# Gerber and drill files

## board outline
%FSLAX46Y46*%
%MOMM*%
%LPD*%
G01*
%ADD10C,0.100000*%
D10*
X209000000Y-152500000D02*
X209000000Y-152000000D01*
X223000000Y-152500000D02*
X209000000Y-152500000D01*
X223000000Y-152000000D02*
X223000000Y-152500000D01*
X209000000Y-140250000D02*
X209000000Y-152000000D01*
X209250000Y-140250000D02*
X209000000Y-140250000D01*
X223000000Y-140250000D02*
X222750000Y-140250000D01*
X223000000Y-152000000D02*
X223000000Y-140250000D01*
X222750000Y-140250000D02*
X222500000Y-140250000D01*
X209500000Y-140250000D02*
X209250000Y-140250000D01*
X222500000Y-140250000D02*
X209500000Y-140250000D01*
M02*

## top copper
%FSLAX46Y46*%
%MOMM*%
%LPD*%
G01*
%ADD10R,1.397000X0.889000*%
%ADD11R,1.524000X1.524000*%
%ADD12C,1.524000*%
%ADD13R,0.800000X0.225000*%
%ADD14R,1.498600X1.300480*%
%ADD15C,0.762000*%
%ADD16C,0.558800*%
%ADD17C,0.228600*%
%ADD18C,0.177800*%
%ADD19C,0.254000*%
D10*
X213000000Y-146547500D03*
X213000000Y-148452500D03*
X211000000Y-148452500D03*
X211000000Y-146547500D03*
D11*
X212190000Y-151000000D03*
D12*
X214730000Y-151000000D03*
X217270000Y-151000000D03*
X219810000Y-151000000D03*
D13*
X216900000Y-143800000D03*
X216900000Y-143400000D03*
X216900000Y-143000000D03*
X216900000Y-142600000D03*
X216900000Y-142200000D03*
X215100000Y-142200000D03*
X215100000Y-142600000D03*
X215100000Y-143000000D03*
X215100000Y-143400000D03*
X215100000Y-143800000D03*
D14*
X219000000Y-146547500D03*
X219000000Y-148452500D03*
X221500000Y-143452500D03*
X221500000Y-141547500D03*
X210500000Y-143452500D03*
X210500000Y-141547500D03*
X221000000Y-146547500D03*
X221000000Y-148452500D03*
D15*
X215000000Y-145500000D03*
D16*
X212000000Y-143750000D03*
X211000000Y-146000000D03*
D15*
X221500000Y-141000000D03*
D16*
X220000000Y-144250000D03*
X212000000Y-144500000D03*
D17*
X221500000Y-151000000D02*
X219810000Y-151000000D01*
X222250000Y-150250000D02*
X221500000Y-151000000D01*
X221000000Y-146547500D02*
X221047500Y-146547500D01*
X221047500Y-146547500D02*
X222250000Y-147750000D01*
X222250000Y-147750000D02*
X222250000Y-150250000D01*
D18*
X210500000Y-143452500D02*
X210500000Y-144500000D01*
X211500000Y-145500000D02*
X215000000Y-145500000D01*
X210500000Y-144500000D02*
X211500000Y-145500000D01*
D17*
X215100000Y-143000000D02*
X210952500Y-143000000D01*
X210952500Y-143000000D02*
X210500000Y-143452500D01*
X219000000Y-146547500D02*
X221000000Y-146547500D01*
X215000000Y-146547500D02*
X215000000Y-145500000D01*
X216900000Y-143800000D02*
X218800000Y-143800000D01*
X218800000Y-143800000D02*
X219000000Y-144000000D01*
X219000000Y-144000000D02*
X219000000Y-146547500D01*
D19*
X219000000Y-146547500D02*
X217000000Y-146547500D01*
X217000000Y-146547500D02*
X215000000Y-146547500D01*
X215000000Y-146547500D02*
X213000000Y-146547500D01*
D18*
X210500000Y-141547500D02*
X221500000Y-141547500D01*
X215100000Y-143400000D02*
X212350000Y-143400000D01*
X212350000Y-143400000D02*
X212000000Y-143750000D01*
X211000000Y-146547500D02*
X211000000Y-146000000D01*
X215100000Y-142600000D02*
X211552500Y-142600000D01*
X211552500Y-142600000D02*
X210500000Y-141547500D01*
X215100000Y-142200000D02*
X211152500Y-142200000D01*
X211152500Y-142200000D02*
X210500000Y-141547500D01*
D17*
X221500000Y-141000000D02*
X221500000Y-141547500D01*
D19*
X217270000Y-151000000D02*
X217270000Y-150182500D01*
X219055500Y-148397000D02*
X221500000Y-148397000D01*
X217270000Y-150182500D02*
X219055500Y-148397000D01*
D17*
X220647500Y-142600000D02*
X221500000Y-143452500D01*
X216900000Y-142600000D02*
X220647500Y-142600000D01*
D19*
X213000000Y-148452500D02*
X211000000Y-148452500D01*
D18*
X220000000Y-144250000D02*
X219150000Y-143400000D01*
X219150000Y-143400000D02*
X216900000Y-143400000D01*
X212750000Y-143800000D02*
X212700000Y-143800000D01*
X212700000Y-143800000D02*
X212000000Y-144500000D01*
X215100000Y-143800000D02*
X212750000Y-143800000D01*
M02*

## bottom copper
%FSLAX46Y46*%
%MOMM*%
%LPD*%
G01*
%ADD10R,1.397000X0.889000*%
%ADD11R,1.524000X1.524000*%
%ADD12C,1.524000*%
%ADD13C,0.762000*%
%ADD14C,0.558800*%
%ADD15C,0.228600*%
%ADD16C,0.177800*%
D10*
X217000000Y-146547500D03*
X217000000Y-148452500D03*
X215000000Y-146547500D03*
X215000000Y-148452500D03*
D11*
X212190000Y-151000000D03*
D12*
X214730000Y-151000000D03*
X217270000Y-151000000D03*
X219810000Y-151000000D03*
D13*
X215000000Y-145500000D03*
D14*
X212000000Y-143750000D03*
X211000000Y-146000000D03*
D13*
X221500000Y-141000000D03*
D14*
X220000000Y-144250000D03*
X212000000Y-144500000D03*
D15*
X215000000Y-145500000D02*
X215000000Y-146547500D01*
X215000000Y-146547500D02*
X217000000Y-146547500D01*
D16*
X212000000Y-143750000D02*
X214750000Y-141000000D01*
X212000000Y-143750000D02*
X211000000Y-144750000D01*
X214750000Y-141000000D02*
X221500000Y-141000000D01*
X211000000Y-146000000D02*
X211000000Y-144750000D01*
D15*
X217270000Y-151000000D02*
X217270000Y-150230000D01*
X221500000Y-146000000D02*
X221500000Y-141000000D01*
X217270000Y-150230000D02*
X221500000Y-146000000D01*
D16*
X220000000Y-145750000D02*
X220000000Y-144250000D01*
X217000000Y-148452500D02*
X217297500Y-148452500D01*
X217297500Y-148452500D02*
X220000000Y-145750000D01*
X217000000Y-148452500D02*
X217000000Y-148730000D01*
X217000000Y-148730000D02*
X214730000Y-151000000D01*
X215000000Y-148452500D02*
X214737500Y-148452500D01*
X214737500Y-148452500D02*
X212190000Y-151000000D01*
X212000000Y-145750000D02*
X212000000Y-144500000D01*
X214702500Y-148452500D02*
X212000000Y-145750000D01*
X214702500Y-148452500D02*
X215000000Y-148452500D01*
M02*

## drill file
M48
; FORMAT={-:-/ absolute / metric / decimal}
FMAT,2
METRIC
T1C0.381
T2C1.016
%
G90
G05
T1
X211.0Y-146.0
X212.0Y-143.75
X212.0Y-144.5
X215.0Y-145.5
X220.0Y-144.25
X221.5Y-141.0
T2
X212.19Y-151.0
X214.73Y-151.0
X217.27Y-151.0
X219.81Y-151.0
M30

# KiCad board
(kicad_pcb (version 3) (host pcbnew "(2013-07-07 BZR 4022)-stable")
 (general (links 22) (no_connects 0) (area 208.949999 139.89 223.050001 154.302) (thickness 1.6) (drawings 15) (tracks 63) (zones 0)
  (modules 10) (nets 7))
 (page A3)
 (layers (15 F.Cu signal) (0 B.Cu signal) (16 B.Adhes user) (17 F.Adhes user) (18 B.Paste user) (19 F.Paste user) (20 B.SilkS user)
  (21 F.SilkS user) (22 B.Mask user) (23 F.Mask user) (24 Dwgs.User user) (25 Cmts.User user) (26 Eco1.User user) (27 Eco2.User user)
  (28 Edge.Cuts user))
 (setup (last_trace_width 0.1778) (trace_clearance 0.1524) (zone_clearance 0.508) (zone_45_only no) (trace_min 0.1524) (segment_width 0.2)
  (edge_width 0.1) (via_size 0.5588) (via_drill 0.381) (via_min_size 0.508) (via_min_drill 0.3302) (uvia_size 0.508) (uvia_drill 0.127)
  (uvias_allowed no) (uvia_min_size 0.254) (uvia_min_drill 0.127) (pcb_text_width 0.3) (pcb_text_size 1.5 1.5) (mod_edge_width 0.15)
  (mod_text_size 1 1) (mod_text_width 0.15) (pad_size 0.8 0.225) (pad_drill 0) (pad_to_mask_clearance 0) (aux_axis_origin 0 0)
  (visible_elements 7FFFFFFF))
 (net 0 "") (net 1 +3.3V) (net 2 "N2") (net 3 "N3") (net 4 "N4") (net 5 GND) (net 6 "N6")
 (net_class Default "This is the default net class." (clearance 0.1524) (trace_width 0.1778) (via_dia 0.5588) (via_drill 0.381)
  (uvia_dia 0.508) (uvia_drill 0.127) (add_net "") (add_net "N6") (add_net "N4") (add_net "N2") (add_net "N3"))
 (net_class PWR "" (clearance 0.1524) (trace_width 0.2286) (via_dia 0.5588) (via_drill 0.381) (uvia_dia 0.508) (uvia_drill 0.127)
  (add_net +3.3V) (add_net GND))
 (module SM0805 (layer B.Cu) (at 217 147.5 270)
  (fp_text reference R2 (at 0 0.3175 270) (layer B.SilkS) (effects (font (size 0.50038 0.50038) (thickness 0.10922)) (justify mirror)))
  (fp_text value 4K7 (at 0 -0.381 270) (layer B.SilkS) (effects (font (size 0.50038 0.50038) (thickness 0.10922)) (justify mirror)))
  (pad 1 smd rect (at -0.9525 0 270) (size 0.889 1.397) (layers B.Cu B.Paste B.Mask) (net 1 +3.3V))
  (pad 2 smd rect (at 0.9525 0 270) (size 0.889 1.397) (layers B.Cu B.Paste B.Mask) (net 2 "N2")))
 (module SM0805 (layer B.Cu) (at 215 147.5 270)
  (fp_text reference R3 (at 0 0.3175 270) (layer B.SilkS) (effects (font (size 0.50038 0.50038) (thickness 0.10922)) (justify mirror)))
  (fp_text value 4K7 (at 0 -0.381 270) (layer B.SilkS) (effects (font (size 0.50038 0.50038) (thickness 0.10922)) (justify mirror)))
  (pad 1 smd rect (at -0.9525 0 270) (size 0.889 1.397) (layers B.Cu B.Paste B.Mask) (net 1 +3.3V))
  (pad 2 smd rect (at 0.9525 0 270) (size 0.889 1.397) (layers B.Cu B.Paste B.Mask) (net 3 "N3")))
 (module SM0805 (layer F.Cu) (at 213 147.5 270)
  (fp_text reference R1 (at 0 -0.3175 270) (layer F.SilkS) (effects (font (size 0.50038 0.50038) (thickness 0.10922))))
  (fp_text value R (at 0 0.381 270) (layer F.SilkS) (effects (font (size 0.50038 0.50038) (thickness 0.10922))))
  (pad 1 smd rect (at -0.9525 0 270) (size 0.889 1.397) (layers F.Cu F.Paste F.Mask) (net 1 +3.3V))
  (pad 2 smd rect (at 0.9525 0 270) (size 0.889 1.397) (layers F.Cu F.Paste F.Mask) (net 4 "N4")))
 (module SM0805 (layer F.Cu) (at 211 147.5 90)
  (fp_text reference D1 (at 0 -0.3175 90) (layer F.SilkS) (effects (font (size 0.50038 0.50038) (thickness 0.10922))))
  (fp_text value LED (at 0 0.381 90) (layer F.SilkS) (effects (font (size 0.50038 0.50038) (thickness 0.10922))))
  (pad 1 smd rect (at -0.9525 0 90) (size 0.889 1.397) (layers F.Cu F.Paste F.Mask) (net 4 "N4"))
  (pad 2 smd rect (at 0.9525 0 90) (size 0.889 1.397) (layers F.Cu F.Paste F.Mask) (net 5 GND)))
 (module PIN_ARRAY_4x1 (layer F.Cu) (at 216 151)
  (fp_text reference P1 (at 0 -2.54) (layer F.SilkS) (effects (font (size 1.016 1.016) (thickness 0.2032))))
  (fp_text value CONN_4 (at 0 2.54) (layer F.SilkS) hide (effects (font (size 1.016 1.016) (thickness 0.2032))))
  (pad 1 thru_hole rect (at -3.81 0) (size 1.524 1.524) (drill 1.016) (layers *.Cu *.Mask F.SilkS) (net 3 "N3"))
  (pad 2 thru_hole circle (at -1.27 0) (size 1.524 1.524) (drill 1.016) (layers *.Cu *.Mask F.SilkS) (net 2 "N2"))
  (pad 3 thru_hole circle (at 1.27 0) (size 1.524 1.524) (drill 1.016) (layers *.Cu *.Mask F.SilkS) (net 5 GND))
  (pad 4 thru_hole circle (at 3.81 0) (size 1.524 1.524) (drill 1.016) (layers *.Cu *.Mask F.SilkS) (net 1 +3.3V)))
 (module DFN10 (layer F.Cu) (at 216 143 180)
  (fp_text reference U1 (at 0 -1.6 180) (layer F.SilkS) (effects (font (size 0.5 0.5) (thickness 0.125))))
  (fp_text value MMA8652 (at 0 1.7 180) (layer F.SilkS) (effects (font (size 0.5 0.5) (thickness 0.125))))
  (pad 1 smd rect (at -0.9 -0.8 180) (size 0.8 0.225) (layers F.Cu F.Paste F.Mask) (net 1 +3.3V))
  (pad 2 smd rect (at -0.9 -0.4 180) (size 0.8 0.225) (layers F.Cu F.Paste F.Mask) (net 2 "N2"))
  (pad 3 smd rect (at -0.9 0 180) (size 0.8 0.225) (layers F.Cu F.Paste F.Mask))
  (pad 4 smd rect (at -0.9 0.4 180) (size 0.8 0.225) (layers F.Cu F.Paste F.Mask) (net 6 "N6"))
  (pad 5 smd rect (at -0.9 0.8 180) (size 0.8 0.225) (layers F.Cu F.Paste F.Mask))
  (pad 6 smd rect (at 0.9 0.8 180) (size 0.8 0.225) (layers F.Cu F.Paste F.Mask) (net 5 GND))
  (pad 7 smd rect (at 0.9 0.4 180) (size 0.8 0.225) (layers F.Cu F.Paste F.Mask) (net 5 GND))
  (pad 8 smd rect (at 0.9 0 180) (size 0.8 0.225) (layers F.Cu F.Paste F.Mask) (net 1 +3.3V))
  (pad 9 smd rect (at 0.9 -0.4 180) (size 0.8 0.225) (layers F.Cu F.Paste F.Mask) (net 5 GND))
  (pad 10 smd rect (at 0.9 -0.8 180) (size 0.8 0.225) (layers F.Cu F.Paste F.Mask) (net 3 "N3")))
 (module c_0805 (layer F.Cu) (at 219 147.5 90)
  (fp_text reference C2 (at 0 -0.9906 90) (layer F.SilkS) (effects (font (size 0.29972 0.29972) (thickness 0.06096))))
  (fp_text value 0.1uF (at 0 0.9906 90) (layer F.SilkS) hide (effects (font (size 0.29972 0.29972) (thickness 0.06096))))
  (pad 1 smd rect (at 0.9525 0 90) (size 1.30048 1.4986) (layers F.Cu F.Paste F.Mask) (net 1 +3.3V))
  (pad 2 smd rect (at -0.9525 0 90) (size 1.30048 1.4986) (layers F.Cu F.Paste F.Mask) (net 5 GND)))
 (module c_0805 (layer F.Cu) (at 221.5 142.5 270)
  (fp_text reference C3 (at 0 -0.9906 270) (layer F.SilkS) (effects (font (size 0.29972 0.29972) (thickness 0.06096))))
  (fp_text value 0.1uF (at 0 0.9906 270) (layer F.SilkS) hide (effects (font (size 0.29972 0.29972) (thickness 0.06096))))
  (pad 1 smd rect (at 0.9525 0 270) (size 1.30048 1.4986) (layers F.Cu F.Paste F.Mask) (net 6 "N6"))
  (pad 2 smd rect (at -0.9525 0 270) (size 1.30048 1.4986) (layers F.Cu F.Paste F.Mask) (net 5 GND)))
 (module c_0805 (layer F.Cu) (at 210.5 142.5 270)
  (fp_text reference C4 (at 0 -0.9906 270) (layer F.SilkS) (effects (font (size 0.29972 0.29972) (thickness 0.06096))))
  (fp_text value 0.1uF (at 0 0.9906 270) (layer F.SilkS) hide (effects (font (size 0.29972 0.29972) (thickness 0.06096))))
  (pad 1 smd rect (at 0.9525 0 270) (size 1.30048 1.4986) (layers F.Cu F.Paste F.Mask) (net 1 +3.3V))
  (pad 2 smd rect (at -0.9525 0 270) (size 1.30048 1.4986) (layers F.Cu F.Paste F.Mask) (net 5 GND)))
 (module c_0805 (layer F.Cu) (at 221 147.5 90)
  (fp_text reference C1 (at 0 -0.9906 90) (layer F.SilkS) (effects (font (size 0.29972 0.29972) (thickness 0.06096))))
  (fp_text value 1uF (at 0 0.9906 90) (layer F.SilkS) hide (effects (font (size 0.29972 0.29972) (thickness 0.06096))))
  (pad 1 smd rect (at 0.9525 0 90) (size 1.30048 1.4986) (layers F.Cu F.Paste F.Mask) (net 1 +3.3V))
  (pad 2 smd rect (at -0.9525 0 90) (size 1.30048 1.4986) (layers F.Cu F.Paste F.Mask) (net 5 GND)))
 (gr_line (start 209 152.5) (end 209 152) (angle 90) (layer Edge.Cuts) (width 0.1))
 (gr_line (start 223 152.5) (end 209 152.5) (angle 90) (layer Edge.Cuts) (width 0.1))
 (gr_line (start 223 152) (end 223 152.5) (angle 90) (layer Edge.Cuts) (width 0.1))
 (gr_line (start 209 140.25) (end 209 152) (angle 90) (layer Edge.Cuts) (width 0.1))
 (gr_line (start 209.25 140.25) (end 209 140.25) (angle 90) (layer Edge.Cuts) (width 0.1))
 (gr_line (start 223 140.25) (end 222.75 140.25) (angle 90) (layer Edge.Cuts) (width 0.1))
 (gr_line (start 223 152) (end 223 140.25) (angle 90) (layer Edge.Cuts) (width 0.1))
 (gr_line (start 222.75 140.25) (end 222.5 140.25) (angle 90) (layer Edge.Cuts) (width 0.1))
 (gr_line (start 209.5 140.25) (end 209.25 140.25) (angle 90) (layer Edge.Cuts) (width 0.1))
 (gr_line (start 222.5 140.25) (end 209.5 140.25) (angle 90) (layer Edge.Cuts) (width 0.1))
 (segment (start 221.5 151) (end 219.81 151) (width 0.2286) (layer F.Cu) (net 1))
 (segment (start 222.25 150.25) (end 221.5 151) (width 0.2286) (layer F.Cu) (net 1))
 (segment (start 221 146.5475) (end 221.0475 146.5475) (width 0.2286) (layer F.Cu) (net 1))
 (segment (start 221.0475 146.5475) (end 222.25 147.75) (width 0.2286) (layer F.Cu) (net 1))
 (segment (start 222.25 147.75) (end 222.25 150.25) (width 0.2286) (layer F.Cu) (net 1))
 (segment (start 210.5 143.4525) (end 210.5 144.5) (width 0.1778) (layer F.Cu) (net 1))
 (segment (start 211.5 145.5) (end 215 145.5) (width 0.1778) (layer F.Cu) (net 1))
 (segment (start 210.5 144.5) (end 211.5 145.5) (width 0.1778) (layer F.Cu) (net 1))
 (segment (start 215.1 143) (end 210.9525 143) (width 0.2286) (layer F.Cu) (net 1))
 (segment (start 210.9525 143) (end 210.5 143.4525) (width 0.2286) (layer F.Cu) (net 1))
 (segment (start 219 146.5475) (end 221 146.5475) (width 0.2286) (layer F.Cu) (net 1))
 (segment (start 215 146.5475) (end 215 145.5) (width 0.2286) (layer F.Cu) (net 1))
 (segment (start 215 145.5) (end 215 146.5475) (width 0.2286) (layer B.Cu) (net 1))
 (via (at 215 145.5) (size 0.762) (layers F.Cu B.Cu) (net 1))
 (segment (start 215 146.5475) (end 217 146.5475) (width 0.2286) (layer B.Cu) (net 1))
 (segment (start 216.9 143.8) (end 218.8 143.8) (width 0.2286) (layer F.Cu) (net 1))
 (segment (start 218.8 143.8) (end 219 144) (width 0.2286) (layer F.Cu) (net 1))
 (segment (start 219 144) (end 219 146.5475) (width 0.2286) (layer F.Cu) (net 1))
 (segment (start 219 146.5475) (end 217 146.5475) (width 0.254) (layer F.Cu) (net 1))
 (segment (start 217 146.5475) (end 215 146.5475) (width 0.254) (layer F.Cu) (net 1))
 (segment (start 215 146.5475) (end 213 146.5475) (width 0.254) (layer F.Cu) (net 1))
 (segment (start 210.5 141.5475) (end 221.5 141.5475) (width 0.1778) (layer F.Cu) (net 5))
 (segment (start 212 143.75) (end 214.75 141) (width 0.1778) (layer B.Cu) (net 5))
 (segment (start 215.1 143.4) (end 212.35 143.4) (width 0.1778) (layer F.Cu) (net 5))
 (segment (start 212 143.75) (end 211 144.75) (width 0.1778) (layer B.Cu) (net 5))
 (via (at 212 143.75) (size 0.5588) (layers F.Cu B.Cu) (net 5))
 (segment (start 212.35 143.4) (end 212 143.75) (width 0.1778) (layer F.Cu) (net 5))
 (segment (start 211 146.5475) (end 211 146) (width 0.1778) (layer F.Cu) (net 5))
 (segment (start 214.75 141) (end 221.5 141) (width 0.1778) (layer B.Cu) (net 5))
 (segment (start 211 146) (end 211 144.75) (width 0.1778) (layer B.Cu) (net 5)) (via (at 211 146) (size 0.5588) (layers F.Cu B.Cu) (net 5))
 (segment (start 215.1 142.6) (end 211.5525 142.6) (width 0.1778) (layer F.Cu) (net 5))
 (segment (start 211.5525 142.6) (end 210.5 141.5475) (width 0.1778) (layer F.Cu) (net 5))
 (segment (start 215.1 142.2) (end 211.1525 142.2) (width 0.1778) (layer F.Cu) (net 5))
 (segment (start 211.1525 142.2) (end 210.5 141.5475) (width 0.1778) (layer F.Cu) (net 5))
 (segment (start 217.27 151) (end 217.27 150.23) (width 0.2286) (layer B.Cu) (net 5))
 (segment (start 221.5 141) (end 221.5 141.5475) (width 0.2286) (layer F.Cu) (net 5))
 (via (at 221.5 141) (size 0.762) (layers F.Cu B.Cu) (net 5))
 (segment (start 221.5 146) (end 221.5 141) (width 0.2286) (layer B.Cu) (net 5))
 (segment (start 217.27 150.23) (end 221.5 146) (width 0.2286) (layer B.Cu) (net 5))
 (segment (start 217.27 151) (end 217.27 150.1825) (width 0.254) (layer F.Cu) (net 5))
 (segment (start 219.0555 148.397) (end 221.5 148.397) (width 0.254) (layer F.Cu) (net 5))
 (segment (start 217.27 150.1825) (end 219.0555 148.397) (width 0.254) (layer F.Cu) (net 5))
 (segment (start 220.6475 142.6) (end 221.5 143.4525) (width 0.2286) (layer F.Cu) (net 6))
 (segment (start 216.9 142.6) (end 220.6475 142.6) (width 0.2286) (layer F.Cu) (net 6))
 (segment (start 213 148.4525) (end 211 148.4525) (width 0.254) (layer F.Cu) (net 4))
 (segment (start 220 144.25) (end 219.15 143.4) (width 0.1778) (layer F.Cu) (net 2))
 (segment (start 220 145.75) (end 220 144.25) (width 0.1778) (layer B.Cu) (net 2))
 (via (at 220 144.25) (size 0.5588) (layers F.Cu B.Cu) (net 2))
 (segment (start 217 148.4525) (end 217.2975 148.4525) (width 0.1778) (layer B.Cu) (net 2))
 (segment (start 217.2975 148.4525) (end 220 145.75) (width 0.1778) (layer B.Cu) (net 2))
 (segment (start 219.15 143.4) (end 216.9 143.4) (width 0.1778) (layer F.Cu) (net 2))
 (segment (start 217 148.4525) (end 217 148.73) (width 0.1778) (layer B.Cu) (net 2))
 (segment (start 217 148.73) (end 214.73 151) (width 0.1778) (layer B.Cu) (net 2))
 (segment (start 215 148.4525) (end 214.7375 148.4525) (width 0.1778) (layer B.Cu) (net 3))
 (segment (start 214.7375 148.4525) (end 212.19 151) (width 0.1778) (layer B.Cu) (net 3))
 (segment (start 212 145.75) (end 212 144.5) (width 0.1778) (layer B.Cu) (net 3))
 (segment (start 212.75 143.8) (end 212.7 143.8) (width 0.1778) (layer F.Cu) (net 3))
 (segment (start 212.7 143.8) (end 212 144.5) (width 0.1778) (layer F.Cu) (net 3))
 (segment (start 215.1 143.8) (end 212.75 143.8) (width 0.1778) (layer F.Cu) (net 3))
 (via (at 212 144.5) (size 0.5588) (layers F.Cu B.Cu) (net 3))
 (segment (start 214.7025 148.4525) (end 212 145.75) (width 0.1778) (layer B.Cu) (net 3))
 (segment (start 214.7025 148.4525) (end 215 148.4525) (width 0.1778) (layer B.Cu) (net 3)))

